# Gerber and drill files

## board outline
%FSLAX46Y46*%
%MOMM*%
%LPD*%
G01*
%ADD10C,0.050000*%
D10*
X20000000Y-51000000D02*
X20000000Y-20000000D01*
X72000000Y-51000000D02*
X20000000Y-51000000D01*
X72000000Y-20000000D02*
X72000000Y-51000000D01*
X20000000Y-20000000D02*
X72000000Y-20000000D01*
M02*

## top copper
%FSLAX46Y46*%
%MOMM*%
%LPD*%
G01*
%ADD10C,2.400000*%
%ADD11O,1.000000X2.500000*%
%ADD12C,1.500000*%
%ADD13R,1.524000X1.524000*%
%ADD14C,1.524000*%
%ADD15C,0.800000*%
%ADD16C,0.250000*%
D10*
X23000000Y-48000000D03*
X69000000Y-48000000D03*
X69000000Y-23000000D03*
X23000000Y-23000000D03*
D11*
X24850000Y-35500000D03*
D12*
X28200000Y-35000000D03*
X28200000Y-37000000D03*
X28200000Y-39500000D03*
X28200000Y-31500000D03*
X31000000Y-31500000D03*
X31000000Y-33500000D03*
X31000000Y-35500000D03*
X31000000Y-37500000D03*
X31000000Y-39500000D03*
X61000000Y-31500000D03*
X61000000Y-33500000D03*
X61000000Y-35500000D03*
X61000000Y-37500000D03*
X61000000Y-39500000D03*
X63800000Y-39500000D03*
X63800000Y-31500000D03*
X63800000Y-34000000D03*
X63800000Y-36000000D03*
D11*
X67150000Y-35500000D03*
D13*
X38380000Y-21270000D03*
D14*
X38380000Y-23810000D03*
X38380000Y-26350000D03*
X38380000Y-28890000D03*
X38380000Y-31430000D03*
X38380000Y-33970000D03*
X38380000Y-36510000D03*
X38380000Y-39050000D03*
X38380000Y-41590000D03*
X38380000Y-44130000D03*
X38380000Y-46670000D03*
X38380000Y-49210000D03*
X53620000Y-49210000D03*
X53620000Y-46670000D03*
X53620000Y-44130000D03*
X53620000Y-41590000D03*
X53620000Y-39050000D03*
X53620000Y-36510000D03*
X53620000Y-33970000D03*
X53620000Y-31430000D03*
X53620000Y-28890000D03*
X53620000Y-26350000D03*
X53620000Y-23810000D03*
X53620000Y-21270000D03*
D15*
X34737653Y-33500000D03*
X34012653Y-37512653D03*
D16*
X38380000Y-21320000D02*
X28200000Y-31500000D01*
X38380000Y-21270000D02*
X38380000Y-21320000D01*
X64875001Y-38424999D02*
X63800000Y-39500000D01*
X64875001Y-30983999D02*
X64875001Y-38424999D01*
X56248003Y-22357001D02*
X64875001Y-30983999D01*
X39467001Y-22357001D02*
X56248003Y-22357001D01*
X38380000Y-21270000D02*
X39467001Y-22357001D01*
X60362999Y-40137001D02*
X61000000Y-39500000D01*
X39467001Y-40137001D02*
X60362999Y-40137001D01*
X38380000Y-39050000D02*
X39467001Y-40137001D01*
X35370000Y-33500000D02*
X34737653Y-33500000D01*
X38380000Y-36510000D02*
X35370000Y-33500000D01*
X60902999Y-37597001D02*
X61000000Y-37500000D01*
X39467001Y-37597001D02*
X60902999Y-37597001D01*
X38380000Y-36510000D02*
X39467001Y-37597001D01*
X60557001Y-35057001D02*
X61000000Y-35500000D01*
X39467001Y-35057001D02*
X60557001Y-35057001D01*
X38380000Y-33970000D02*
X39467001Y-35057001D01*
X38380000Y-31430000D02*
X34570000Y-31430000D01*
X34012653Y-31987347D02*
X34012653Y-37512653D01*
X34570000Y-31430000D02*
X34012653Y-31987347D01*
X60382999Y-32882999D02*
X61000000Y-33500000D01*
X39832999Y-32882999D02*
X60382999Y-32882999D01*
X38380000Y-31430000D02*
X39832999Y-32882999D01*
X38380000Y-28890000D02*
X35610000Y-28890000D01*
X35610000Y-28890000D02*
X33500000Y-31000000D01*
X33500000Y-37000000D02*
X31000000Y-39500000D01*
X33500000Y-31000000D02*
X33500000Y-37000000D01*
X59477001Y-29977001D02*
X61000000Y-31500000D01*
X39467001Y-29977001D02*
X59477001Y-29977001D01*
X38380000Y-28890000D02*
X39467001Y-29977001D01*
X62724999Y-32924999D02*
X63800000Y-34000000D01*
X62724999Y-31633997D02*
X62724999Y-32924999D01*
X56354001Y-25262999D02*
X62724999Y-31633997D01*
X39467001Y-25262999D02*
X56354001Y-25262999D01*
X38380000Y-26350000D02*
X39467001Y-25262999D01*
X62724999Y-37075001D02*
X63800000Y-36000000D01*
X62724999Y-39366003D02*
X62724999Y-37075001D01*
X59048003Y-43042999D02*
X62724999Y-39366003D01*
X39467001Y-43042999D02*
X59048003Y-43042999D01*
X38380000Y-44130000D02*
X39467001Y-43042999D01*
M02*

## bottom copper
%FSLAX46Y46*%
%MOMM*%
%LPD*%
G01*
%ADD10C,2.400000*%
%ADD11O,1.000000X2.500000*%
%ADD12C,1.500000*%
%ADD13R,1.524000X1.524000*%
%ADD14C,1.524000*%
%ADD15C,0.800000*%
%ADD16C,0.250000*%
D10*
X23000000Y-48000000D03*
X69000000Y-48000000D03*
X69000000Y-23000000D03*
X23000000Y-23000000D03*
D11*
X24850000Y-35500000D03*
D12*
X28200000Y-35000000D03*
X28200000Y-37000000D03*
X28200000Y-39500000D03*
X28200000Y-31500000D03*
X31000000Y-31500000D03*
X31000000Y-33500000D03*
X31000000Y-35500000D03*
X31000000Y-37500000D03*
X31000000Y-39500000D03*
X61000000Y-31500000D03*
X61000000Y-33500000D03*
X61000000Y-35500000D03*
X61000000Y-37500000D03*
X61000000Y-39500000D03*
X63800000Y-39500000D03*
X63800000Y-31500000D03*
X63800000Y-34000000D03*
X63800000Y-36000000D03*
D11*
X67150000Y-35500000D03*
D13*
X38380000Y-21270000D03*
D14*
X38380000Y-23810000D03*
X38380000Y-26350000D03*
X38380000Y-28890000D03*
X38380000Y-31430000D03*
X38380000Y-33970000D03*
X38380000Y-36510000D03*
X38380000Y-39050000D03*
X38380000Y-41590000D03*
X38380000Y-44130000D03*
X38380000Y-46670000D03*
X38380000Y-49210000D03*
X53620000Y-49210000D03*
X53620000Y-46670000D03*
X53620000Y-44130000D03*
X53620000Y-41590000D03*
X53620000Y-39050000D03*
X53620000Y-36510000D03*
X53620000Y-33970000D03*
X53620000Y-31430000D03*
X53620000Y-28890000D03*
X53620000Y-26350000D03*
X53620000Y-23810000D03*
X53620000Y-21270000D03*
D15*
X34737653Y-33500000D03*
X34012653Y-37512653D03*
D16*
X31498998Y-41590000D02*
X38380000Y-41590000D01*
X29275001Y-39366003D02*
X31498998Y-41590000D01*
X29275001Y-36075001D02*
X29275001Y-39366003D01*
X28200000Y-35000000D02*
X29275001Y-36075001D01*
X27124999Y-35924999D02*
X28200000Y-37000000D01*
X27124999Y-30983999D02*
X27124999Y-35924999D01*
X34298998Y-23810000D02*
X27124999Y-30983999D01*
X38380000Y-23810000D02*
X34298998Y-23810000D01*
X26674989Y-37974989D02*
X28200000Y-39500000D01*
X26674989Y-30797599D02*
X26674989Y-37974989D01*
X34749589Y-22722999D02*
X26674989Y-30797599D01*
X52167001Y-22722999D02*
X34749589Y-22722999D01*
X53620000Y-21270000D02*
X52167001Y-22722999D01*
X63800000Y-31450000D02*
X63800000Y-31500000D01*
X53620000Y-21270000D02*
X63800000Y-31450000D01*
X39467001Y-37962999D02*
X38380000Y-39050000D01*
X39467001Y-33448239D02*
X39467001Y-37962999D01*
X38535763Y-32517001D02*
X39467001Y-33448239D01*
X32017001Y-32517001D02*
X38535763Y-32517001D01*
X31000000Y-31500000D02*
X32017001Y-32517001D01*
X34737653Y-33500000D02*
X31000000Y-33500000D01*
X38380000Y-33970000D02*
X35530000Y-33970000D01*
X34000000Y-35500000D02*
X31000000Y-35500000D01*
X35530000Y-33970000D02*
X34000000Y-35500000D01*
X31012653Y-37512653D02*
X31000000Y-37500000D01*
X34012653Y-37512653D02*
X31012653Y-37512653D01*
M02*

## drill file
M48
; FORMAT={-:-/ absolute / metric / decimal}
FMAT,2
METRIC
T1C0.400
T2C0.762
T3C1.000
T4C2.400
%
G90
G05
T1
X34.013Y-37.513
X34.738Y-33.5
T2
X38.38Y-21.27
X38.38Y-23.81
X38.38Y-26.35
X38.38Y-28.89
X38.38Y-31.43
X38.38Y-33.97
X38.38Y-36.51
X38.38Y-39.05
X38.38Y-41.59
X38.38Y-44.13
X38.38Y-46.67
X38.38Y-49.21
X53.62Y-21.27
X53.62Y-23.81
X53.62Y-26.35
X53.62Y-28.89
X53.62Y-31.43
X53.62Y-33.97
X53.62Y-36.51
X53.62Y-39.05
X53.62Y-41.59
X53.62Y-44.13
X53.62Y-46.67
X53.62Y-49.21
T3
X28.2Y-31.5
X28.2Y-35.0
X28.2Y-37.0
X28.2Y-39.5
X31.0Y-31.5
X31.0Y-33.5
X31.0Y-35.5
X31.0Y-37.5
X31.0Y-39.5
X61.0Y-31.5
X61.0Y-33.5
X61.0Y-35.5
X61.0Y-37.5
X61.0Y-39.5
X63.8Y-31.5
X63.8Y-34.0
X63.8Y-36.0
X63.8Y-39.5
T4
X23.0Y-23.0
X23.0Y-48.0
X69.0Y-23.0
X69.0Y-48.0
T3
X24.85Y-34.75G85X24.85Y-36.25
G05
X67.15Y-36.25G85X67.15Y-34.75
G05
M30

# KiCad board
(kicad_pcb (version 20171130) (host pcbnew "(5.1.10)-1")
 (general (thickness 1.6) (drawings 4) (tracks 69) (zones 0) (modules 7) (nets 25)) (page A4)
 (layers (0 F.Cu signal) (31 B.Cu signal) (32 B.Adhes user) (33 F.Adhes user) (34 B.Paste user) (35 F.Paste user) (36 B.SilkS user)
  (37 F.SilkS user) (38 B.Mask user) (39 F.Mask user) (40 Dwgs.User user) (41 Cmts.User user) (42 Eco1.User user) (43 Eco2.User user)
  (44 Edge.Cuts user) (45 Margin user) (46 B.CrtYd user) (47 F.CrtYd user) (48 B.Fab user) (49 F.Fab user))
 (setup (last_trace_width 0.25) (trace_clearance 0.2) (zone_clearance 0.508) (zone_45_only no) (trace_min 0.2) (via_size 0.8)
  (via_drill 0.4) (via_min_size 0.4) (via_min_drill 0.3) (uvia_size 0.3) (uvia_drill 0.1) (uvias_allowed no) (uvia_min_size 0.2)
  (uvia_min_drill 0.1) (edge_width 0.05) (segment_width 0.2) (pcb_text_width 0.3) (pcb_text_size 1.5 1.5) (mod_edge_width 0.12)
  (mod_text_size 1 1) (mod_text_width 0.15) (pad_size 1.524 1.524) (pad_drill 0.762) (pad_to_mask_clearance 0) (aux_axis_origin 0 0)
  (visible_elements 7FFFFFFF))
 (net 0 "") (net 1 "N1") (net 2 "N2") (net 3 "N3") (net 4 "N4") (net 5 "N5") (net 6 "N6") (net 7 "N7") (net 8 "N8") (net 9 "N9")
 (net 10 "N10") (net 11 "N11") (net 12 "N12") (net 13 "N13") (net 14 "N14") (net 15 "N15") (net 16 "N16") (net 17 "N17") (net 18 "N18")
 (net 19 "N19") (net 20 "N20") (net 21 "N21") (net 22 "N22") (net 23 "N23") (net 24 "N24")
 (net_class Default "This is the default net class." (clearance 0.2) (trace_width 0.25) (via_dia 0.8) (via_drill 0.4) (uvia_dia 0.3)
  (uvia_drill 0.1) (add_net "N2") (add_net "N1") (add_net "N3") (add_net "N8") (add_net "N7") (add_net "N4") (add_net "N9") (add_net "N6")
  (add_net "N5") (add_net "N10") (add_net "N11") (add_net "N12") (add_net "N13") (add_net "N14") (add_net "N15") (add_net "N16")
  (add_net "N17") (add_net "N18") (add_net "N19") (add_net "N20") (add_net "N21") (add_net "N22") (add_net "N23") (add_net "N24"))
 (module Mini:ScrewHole (layer F.Cu) (at 23 48)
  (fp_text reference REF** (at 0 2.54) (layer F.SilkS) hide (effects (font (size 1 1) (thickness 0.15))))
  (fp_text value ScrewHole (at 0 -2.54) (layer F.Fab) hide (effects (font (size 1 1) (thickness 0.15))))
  (pad HOLE thru_hole circle (at 0 0) (size 2.4 2.4) (drill 2.4) (layers *.Cu *.Mask)))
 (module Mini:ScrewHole (layer F.Cu) (at 69 48)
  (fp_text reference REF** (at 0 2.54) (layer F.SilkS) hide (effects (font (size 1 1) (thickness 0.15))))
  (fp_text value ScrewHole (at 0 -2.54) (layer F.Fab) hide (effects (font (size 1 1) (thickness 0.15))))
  (pad HOLE thru_hole circle (at 0 0) (size 2.4 2.4) (drill 2.4) (layers *.Cu *.Mask)))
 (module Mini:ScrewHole (layer F.Cu) (at 69 23)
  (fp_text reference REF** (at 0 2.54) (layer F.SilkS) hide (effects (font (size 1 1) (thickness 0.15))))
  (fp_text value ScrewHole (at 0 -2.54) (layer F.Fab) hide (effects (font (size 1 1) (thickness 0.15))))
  (pad HOLE thru_hole circle (at 0 0) (size 2.4 2.4) (drill 2.4) (layers *.Cu *.Mask)))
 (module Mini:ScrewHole (layer F.Cu) (at 23 23)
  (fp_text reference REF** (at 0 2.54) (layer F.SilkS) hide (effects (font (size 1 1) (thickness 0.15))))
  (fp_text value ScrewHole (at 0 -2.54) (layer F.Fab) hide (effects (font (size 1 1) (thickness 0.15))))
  (pad HOLE thru_hole circle (at 0 0) (size 2.4 2.4) (drill 2.4) (layers *.Cu *.Mask)))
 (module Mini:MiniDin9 (layer F.Cu) (at 24.85 35.5 270)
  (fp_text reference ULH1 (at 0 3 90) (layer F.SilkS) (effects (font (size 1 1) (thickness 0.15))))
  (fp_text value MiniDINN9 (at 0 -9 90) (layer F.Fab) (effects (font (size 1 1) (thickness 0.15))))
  (pad HOLE thru_hole oval (at 0 0 270) (size 2.5 1) (drill oval 2.5 1) (layers *.Cu *.Mask))
  (pad 2 thru_hole circle (at -0.5 -3.35 270) (size 1.5 1.5) (drill 1) (layers *.Cu *.Mask) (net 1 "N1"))
  (pad 1 thru_hole circle (at 1.5 -3.35 270) (size 1.5 1.5) (drill 1) (layers *.Cu *.Mask) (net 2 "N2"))
  (pad 3 thru_hole circle (at 4 -3.35 270) (size 1.5 1.5) (drill 1) (layers *.Cu *.Mask) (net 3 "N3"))
  (pad 6 thru_hole circle (at -4 -3.35 270) (size 1.5 1.5) (drill 1) (layers *.Cu *.Mask) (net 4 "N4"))
  (pad 9 thru_hole circle (at -4 -6.15 270) (size 1.5 1.5) (drill 1) (layers *.Cu *.Mask) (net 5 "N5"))
  (pad 8 thru_hole circle (at -2 -6.15 270) (size 1.5 1.5) (drill 1) (layers *.Cu *.Mask) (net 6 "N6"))
  (pad 5 thru_hole circle (at 0 -6.15 270) (size 1.5 1.5) (drill 1) (layers *.Cu *.Mask) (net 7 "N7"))
  (pad 4 thru_hole circle (at 2 -6.15 270) (size 1.5 1.5) (drill 1) (layers *.Cu *.Mask) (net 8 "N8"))
  (pad 7 thru_hole circle (at 4 -6.15 270) (size 1.5 1.5) (drill 1) (layers *.Cu *.Mask) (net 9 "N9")))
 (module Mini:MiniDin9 (layer F.Cu) (at 67.15 35.5 90)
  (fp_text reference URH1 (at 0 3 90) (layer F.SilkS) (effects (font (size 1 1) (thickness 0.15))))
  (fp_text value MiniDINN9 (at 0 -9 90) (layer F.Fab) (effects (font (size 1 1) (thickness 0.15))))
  (pad 7 thru_hole circle (at 4 -6.15 90) (size 1.5 1.5) (drill 1) (layers *.Cu *.Mask) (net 9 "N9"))
  (pad 4 thru_hole circle (at 2 -6.15 90) (size 1.5 1.5) (drill 1) (layers *.Cu *.Mask) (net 8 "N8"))
  (pad 5 thru_hole circle (at 0 -6.15 90) (size 1.5 1.5) (drill 1) (layers *.Cu *.Mask) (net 7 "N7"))
  (pad 8 thru_hole circle (at -2 -6.15 90) (size 1.5 1.5) (drill 1) (layers *.Cu *.Mask) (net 6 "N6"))
  (pad 9 thru_hole circle (at -4 -6.15 90) (size 1.5 1.5) (drill 1) (layers *.Cu *.Mask) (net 5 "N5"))
  (pad 6 thru_hole circle (at -4 -3.35 90) (size 1.5 1.5) (drill 1) (layers *.Cu *.Mask) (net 4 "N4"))
  (pad 3 thru_hole circle (at 4 -3.35 90) (size 1.5 1.5) (drill 1) (layers *.Cu *.Mask) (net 3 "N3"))
  (pad 1 thru_hole circle (at 1.5 -3.35 90) (size 1.5 1.5) (drill 1) (layers *.Cu *.Mask) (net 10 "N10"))
  (pad 2 thru_hole circle (at -0.5 -3.35 90) (size 1.5 1.5) (drill 1) (layers *.Cu *.Mask) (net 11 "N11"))
  (pad HOLE thru_hole oval (at 0 0 90) (size 2.5 1) (drill oval 2.5 1) (layers *.Cu *.Mask)))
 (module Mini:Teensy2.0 (layer F.Cu) (at 46 35.24)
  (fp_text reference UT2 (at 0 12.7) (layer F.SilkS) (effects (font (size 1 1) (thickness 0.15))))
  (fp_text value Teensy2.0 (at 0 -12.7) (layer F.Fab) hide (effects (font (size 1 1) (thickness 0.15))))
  (pad 1 thru_hole rect (at -7.62 -13.97) (size 1.524 1.524) (drill 0.762) (layers *.Cu *.Mask) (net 4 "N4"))
  (pad 2 thru_hole circle (at -7.62 -11.43) (size 1.524 1.524) (drill 0.762) (layers *.Cu *.Mask) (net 2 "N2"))
  (pad 3 thru_hole circle (at -7.62 -8.89) (size 1.524 1.524) (drill 0.762) (layers *.Cu *.Mask) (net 10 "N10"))
  (pad 4 thru_hole circle (at -7.62 -6.35) (size 1.524 1.524) (drill 0.762) (layers *.Cu *.Mask) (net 9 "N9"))
  (pad 5 thru_hole circle (at -7.62 -3.81) (size 1.524 1.524) (drill 0.762) (layers *.Cu *.Mask) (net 8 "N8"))
  (pad 6 thru_hole circle (at -7.62 -1.27) (size 1.524 1.524) (drill 0.762) (layers *.Cu *.Mask) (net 7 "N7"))
  (pad 7 thru_hole circle (at -7.62 1.27) (size 1.524 1.524) (drill 0.762) (layers *.Cu *.Mask) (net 6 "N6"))
  (pad 8 thru_hole circle (at -7.62 3.81) (size 1.524 1.524) (drill 0.762) (layers *.Cu *.Mask) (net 5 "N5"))
  (pad 9 thru_hole circle (at -7.62 6.35) (size 1.524 1.524) (drill 0.762) (layers *.Cu *.Mask) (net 1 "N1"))
  (pad 10 thru_hole circle (at -7.62 8.89) (size 1.524 1.524) (drill 0.762) (layers *.Cu *.Mask) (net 11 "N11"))
  (pad 11 thru_hole circle (at -7.62 11.43) (size 1.524 1.524) (drill 0.762) (layers *.Cu *.Mask) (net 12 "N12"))
  (pad 12 thru_hole circle (at -7.62 13.97) (size 1.524 1.524) (drill 0.762) (layers *.Cu *.Mask) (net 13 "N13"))
  (pad 13 thru_hole circle (at 7.62 13.97) (size 1.524 1.524) (drill 0.762) (layers *.Cu *.Mask) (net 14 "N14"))
  (pad 14 thru_hole circle (at 7.62 11.43) (size 1.524 1.524) (drill 0.762) (layers *.Cu *.Mask) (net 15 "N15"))
  (pad 15 thru_hole circle (at 7.62 8.89) (size 1.524 1.524) (drill 0.762) (layers *.Cu *.Mask) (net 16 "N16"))
  (pad 16 thru_hole circle (at 7.62 6.35) (size 1.524 1.524) (drill 0.762) (layers *.Cu *.Mask) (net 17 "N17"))
  (pad 17 thru_hole circle (at 7.62 3.81) (size 1.524 1.524) (drill 0.762) (layers *.Cu *.Mask) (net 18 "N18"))
  (pad 18 thru_hole circle (at 7.62 1.27) (size 1.524 1.524) (drill 0.762) (layers *.Cu *.Mask) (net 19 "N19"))
  (pad 19 thru_hole circle (at 7.62 -1.27) (size 1.524 1.524) (drill 0.762) (layers *.Cu *.Mask) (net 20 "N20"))
  (pad 20 thru_hole circle (at 7.62 -3.81) (size 1.524 1.524) (drill 0.762) (layers *.Cu *.Mask) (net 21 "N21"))
  (pad 21 thru_hole circle (at 7.62 -6.35) (size 1.524 1.524) (drill 0.762) (layers *.Cu *.Mask) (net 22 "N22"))
  (pad 22 thru_hole circle (at 7.62 -8.89) (size 1.524 1.524) (drill 0.762) (layers *.Cu *.Mask) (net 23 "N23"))
  (pad 23 thru_hole circle (at 7.62 -11.43) (size 1.524 1.524) (drill 0.762) (layers *.Cu *.Mask) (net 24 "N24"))
  (pad 24 thru_hole circle (at 7.62 -13.97) (size 1.524 1.524) (drill 0.762) (layers *.Cu *.Mask) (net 3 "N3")))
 (gr_line (start 20 51) (end 20 20) (layer Edge.Cuts) (width 0.05))
 (gr_line (start 72 51) (end 20 51) (layer Edge.Cuts) (width 0.05))
 (gr_line (start 72 20) (end 72 51) (layer Edge.Cuts) (width 0.05))
 (gr_line (start 20 20) (end 72 20) (layer Edge.Cuts) (width 0.05))
 (segment (start 31.498998 41.59) (end 38.38 41.59) (width 0.25) (layer B.Cu) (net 1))
 (segment (start 29.275001 39.366003) (end 31.498998 41.59) (width 0.25) (layer B.Cu) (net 1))
 (segment (start 29.275001 36.075001) (end 29.275001 39.366003) (width 0.25) (layer B.Cu) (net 1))
 (segment (start 28.2 35) (end 29.275001 36.075001) (width 0.25) (layer B.Cu) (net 1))
 (segment (start 27.124999 35.924999) (end 28.2 37) (width 0.25) (layer B.Cu) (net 2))
 (segment (start 27.124999 30.983999) (end 27.124999 35.924999) (width 0.25) (layer B.Cu) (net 2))
 (segment (start 34.298998 23.81) (end 27.124999 30.983999) (width 0.25) (layer B.Cu) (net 2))
 (segment (start 38.38 23.81) (end 34.298998 23.81) (width 0.25) (layer B.Cu) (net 2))
 (segment (start 26.674989 37.974989) (end 28.2 39.5) (width 0.25) (layer B.Cu) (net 3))
 (segment (start 26.674989 30.797599) (end 26.674989 37.974989) (width 0.25) (layer B.Cu) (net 3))
 (segment (start 34.749589 22.722999) (end 26.674989 30.797599) (width 0.25) (layer B.Cu) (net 3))
 (segment (start 52.167001 22.722999) (end 34.749589 22.722999) (width 0.25) (layer B.Cu) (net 3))
 (segment (start 53.62 21.27) (end 52.167001 22.722999) (width 0.25) (layer B.Cu) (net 3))
 (segment (start 63.8 31.45) (end 63.8 31.5) (width 0.25) (layer B.Cu) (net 3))
 (segment (start 53.62 21.27) (end 63.8 31.45) (width 0.25) (layer B.Cu) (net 3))
 (segment (start 38.38 21.32) (end 28.2 31.5) (width 0.25) (layer F.Cu) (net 4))
 (segment (start 38.38 21.27) (end 38.38 21.32) (width 0.25) (layer F.Cu) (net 4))
 (segment (start 64.875001 38.424999) (end 63.8 39.5) (width 0.25) (layer F.Cu) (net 4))
 (segment (start 64.875001 30.983999) (end 64.875001 38.424999) (width 0.25) (layer F.Cu) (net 4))
 (segment (start 56.248003 22.357001) (end 64.875001 30.983999) (width 0.25) (layer F.Cu) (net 4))
 (segment (start 39.467001 22.357001) (end 56.248003 22.357001) (width 0.25) (layer F.Cu) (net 4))
 (segment (start 38.38 21.27) (end 39.467001 22.357001) (width 0.25) (layer F.Cu) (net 4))
 (segment (start 39.467001 37.962999) (end 38.38 39.05) (width 0.25) (layer B.Cu) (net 5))
 (segment (start 39.467001 33.448239) (end 39.467001 37.962999) (width 0.25) (layer B.Cu) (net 5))
 (segment (start 38.535763 32.517001) (end 39.467001 33.448239) (width 0.25) (layer B.Cu) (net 5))
 (segment (start 32.017001 32.517001) (end 38.535763 32.517001) (width 0.25) (layer B.Cu) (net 5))
 (segment (start 31 31.5) (end 32.017001 32.517001) (width 0.25) (layer B.Cu) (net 5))
 (segment (start 60.362999 40.137001) (end 61 39.5) (width 0.25) (layer F.Cu) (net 5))
 (segment (start 39.467001 40.137001) (end 60.362999 40.137001) (width 0.25) (layer F.Cu) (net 5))
 (segment (start 38.38 39.05) (end 39.467001 40.137001) (width 0.25) (layer F.Cu) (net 5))
 (via (at 34.737653 33.5) (size 0.8) (drill 0.4) (layers F.Cu B.Cu) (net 6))
 (segment (start 35.37 33.5) (end 34.737653 33.5) (width 0.25) (layer F.Cu) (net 6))
 (segment (start 38.38 36.51) (end 35.37 33.5) (width 0.25) (layer F.Cu) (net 6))
 (segment (start 34.737653 33.5) (end 31 33.5) (width 0.25) (layer B.Cu) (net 6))
 (segment (start 60.902999 37.597001) (end 61 37.5) (width 0.25) (layer F.Cu) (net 6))
 (segment (start 39.467001 37.597001) (end 60.902999 37.597001) (width 0.25) (layer F.Cu) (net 6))
 (segment (start 38.38 36.51) (end 39.467001 37.597001) (width 0.25) (layer F.Cu) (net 6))
 (segment (start 38.38 33.97) (end 35.53 33.97) (width 0.25) (layer B.Cu) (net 7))
 (segment (start 34 35.5) (end 31 35.5) (width 0.25) (layer B.Cu) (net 7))
 (segment (start 35.53 33.97) (end 34 35.5) (width 0.25) (layer B.Cu) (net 7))
 (segment (start 60.557001 35.057001) (end 61 35.5) (width 0.25) (layer F.Cu) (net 7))
 (segment (start 39.467001 35.057001) (end 60.557001 35.057001) (width 0.25) (layer F.Cu) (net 7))
 (segment (start 38.38 33.97) (end 39.467001 35.057001) (width 0.25) (layer F.Cu) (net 7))
 (segment (start 38.38 31.43) (end 34.57 31.43) (width 0.25) (layer F.Cu) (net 8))
 (via (at 34.012653 37.512653) (size 0.8) (drill 0.4) (layers F.Cu B.Cu) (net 8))
 (segment (start 34.012653 31.987347) (end 34.012653 37.512653) (width 0.25) (layer F.Cu) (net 8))
 (segment (start 34.57 31.43) (end 34.012653 31.987347) (width 0.25) (layer F.Cu) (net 8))
 (segment (start 31.012653 37.512653) (end 31 37.5) (width 0.25) (layer B.Cu) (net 8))
 (segment (start 34.012653 37.512653) (end 31.012653 37.512653) (width 0.25) (layer B.Cu) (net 8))
 (segment (start 60.382999 32.882999) (end 61 33.5) (width 0.25) (layer F.Cu) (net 8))
 (segment (start 39.832999 32.882999) (end 60.382999 32.882999) (width 0.25) (layer F.Cu) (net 8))
 (segment (start 38.38 31.43) (end 39.832999 32.882999) (width 0.25) (layer F.Cu) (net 8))
 (segment (start 38.38 28.89) (end 35.61 28.89) (width 0.25) (layer F.Cu) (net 9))
 (segment (start 35.61 28.89) (end 33.5 31) (width 0.25) (layer F.Cu) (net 9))
 (segment (start 33.5 37) (end 31 39.5) (width 0.25) (layer F.Cu) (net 9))
 (segment (start 33.5 31) (end 33.5 37) (width 0.25) (layer F.Cu) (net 9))
 (segment (start 59.477001 29.977001) (end 61 31.5) (width 0.25) (layer F.Cu) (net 9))
 (segment (start 39.467001 29.977001) (end 59.477001 29.977001) (width 0.25) (layer F.Cu) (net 9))
 (segment (start 38.38 28.89) (end 39.467001 29.977001) (width 0.25) (layer F.Cu) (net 9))
 (segment (start 62.724999 32.924999) (end 63.8 34) (width 0.25) (layer F.Cu) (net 10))
 (segment (start 62.724999 31.633997) (end 62.724999 32.924999) (width 0.25) (layer F.Cu) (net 10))
 (segment (start 56.354001 25.262999) (end 62.724999 31.633997) (width 0.25) (layer F.Cu) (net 10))
 (segment (start 39.467001 25.262999) (end 56.354001 25.262999) (width 0.25) (layer F.Cu) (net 10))
 (segment (start 38.38 26.35) (end 39.467001 25.262999) (width 0.25) (layer F.Cu) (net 10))
 (segment (start 62.724999 37.075001) (end 63.8 36) (width 0.25) (layer F.Cu) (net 11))
 (segment (start 62.724999 39.366003) (end 62.724999 37.075001) (width 0.25) (layer F.Cu) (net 11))
 (segment (start 59.048003 43.042999) (end 62.724999 39.366003) (width 0.25) (layer F.Cu) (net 11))
 (segment (start 39.467001 43.042999) (end 59.048003 43.042999) (width 0.25) (layer F.Cu) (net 11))
 (segment (start 38.38 44.13) (end 39.467001 43.042999) (width 0.25) (layer F.Cu) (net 11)))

